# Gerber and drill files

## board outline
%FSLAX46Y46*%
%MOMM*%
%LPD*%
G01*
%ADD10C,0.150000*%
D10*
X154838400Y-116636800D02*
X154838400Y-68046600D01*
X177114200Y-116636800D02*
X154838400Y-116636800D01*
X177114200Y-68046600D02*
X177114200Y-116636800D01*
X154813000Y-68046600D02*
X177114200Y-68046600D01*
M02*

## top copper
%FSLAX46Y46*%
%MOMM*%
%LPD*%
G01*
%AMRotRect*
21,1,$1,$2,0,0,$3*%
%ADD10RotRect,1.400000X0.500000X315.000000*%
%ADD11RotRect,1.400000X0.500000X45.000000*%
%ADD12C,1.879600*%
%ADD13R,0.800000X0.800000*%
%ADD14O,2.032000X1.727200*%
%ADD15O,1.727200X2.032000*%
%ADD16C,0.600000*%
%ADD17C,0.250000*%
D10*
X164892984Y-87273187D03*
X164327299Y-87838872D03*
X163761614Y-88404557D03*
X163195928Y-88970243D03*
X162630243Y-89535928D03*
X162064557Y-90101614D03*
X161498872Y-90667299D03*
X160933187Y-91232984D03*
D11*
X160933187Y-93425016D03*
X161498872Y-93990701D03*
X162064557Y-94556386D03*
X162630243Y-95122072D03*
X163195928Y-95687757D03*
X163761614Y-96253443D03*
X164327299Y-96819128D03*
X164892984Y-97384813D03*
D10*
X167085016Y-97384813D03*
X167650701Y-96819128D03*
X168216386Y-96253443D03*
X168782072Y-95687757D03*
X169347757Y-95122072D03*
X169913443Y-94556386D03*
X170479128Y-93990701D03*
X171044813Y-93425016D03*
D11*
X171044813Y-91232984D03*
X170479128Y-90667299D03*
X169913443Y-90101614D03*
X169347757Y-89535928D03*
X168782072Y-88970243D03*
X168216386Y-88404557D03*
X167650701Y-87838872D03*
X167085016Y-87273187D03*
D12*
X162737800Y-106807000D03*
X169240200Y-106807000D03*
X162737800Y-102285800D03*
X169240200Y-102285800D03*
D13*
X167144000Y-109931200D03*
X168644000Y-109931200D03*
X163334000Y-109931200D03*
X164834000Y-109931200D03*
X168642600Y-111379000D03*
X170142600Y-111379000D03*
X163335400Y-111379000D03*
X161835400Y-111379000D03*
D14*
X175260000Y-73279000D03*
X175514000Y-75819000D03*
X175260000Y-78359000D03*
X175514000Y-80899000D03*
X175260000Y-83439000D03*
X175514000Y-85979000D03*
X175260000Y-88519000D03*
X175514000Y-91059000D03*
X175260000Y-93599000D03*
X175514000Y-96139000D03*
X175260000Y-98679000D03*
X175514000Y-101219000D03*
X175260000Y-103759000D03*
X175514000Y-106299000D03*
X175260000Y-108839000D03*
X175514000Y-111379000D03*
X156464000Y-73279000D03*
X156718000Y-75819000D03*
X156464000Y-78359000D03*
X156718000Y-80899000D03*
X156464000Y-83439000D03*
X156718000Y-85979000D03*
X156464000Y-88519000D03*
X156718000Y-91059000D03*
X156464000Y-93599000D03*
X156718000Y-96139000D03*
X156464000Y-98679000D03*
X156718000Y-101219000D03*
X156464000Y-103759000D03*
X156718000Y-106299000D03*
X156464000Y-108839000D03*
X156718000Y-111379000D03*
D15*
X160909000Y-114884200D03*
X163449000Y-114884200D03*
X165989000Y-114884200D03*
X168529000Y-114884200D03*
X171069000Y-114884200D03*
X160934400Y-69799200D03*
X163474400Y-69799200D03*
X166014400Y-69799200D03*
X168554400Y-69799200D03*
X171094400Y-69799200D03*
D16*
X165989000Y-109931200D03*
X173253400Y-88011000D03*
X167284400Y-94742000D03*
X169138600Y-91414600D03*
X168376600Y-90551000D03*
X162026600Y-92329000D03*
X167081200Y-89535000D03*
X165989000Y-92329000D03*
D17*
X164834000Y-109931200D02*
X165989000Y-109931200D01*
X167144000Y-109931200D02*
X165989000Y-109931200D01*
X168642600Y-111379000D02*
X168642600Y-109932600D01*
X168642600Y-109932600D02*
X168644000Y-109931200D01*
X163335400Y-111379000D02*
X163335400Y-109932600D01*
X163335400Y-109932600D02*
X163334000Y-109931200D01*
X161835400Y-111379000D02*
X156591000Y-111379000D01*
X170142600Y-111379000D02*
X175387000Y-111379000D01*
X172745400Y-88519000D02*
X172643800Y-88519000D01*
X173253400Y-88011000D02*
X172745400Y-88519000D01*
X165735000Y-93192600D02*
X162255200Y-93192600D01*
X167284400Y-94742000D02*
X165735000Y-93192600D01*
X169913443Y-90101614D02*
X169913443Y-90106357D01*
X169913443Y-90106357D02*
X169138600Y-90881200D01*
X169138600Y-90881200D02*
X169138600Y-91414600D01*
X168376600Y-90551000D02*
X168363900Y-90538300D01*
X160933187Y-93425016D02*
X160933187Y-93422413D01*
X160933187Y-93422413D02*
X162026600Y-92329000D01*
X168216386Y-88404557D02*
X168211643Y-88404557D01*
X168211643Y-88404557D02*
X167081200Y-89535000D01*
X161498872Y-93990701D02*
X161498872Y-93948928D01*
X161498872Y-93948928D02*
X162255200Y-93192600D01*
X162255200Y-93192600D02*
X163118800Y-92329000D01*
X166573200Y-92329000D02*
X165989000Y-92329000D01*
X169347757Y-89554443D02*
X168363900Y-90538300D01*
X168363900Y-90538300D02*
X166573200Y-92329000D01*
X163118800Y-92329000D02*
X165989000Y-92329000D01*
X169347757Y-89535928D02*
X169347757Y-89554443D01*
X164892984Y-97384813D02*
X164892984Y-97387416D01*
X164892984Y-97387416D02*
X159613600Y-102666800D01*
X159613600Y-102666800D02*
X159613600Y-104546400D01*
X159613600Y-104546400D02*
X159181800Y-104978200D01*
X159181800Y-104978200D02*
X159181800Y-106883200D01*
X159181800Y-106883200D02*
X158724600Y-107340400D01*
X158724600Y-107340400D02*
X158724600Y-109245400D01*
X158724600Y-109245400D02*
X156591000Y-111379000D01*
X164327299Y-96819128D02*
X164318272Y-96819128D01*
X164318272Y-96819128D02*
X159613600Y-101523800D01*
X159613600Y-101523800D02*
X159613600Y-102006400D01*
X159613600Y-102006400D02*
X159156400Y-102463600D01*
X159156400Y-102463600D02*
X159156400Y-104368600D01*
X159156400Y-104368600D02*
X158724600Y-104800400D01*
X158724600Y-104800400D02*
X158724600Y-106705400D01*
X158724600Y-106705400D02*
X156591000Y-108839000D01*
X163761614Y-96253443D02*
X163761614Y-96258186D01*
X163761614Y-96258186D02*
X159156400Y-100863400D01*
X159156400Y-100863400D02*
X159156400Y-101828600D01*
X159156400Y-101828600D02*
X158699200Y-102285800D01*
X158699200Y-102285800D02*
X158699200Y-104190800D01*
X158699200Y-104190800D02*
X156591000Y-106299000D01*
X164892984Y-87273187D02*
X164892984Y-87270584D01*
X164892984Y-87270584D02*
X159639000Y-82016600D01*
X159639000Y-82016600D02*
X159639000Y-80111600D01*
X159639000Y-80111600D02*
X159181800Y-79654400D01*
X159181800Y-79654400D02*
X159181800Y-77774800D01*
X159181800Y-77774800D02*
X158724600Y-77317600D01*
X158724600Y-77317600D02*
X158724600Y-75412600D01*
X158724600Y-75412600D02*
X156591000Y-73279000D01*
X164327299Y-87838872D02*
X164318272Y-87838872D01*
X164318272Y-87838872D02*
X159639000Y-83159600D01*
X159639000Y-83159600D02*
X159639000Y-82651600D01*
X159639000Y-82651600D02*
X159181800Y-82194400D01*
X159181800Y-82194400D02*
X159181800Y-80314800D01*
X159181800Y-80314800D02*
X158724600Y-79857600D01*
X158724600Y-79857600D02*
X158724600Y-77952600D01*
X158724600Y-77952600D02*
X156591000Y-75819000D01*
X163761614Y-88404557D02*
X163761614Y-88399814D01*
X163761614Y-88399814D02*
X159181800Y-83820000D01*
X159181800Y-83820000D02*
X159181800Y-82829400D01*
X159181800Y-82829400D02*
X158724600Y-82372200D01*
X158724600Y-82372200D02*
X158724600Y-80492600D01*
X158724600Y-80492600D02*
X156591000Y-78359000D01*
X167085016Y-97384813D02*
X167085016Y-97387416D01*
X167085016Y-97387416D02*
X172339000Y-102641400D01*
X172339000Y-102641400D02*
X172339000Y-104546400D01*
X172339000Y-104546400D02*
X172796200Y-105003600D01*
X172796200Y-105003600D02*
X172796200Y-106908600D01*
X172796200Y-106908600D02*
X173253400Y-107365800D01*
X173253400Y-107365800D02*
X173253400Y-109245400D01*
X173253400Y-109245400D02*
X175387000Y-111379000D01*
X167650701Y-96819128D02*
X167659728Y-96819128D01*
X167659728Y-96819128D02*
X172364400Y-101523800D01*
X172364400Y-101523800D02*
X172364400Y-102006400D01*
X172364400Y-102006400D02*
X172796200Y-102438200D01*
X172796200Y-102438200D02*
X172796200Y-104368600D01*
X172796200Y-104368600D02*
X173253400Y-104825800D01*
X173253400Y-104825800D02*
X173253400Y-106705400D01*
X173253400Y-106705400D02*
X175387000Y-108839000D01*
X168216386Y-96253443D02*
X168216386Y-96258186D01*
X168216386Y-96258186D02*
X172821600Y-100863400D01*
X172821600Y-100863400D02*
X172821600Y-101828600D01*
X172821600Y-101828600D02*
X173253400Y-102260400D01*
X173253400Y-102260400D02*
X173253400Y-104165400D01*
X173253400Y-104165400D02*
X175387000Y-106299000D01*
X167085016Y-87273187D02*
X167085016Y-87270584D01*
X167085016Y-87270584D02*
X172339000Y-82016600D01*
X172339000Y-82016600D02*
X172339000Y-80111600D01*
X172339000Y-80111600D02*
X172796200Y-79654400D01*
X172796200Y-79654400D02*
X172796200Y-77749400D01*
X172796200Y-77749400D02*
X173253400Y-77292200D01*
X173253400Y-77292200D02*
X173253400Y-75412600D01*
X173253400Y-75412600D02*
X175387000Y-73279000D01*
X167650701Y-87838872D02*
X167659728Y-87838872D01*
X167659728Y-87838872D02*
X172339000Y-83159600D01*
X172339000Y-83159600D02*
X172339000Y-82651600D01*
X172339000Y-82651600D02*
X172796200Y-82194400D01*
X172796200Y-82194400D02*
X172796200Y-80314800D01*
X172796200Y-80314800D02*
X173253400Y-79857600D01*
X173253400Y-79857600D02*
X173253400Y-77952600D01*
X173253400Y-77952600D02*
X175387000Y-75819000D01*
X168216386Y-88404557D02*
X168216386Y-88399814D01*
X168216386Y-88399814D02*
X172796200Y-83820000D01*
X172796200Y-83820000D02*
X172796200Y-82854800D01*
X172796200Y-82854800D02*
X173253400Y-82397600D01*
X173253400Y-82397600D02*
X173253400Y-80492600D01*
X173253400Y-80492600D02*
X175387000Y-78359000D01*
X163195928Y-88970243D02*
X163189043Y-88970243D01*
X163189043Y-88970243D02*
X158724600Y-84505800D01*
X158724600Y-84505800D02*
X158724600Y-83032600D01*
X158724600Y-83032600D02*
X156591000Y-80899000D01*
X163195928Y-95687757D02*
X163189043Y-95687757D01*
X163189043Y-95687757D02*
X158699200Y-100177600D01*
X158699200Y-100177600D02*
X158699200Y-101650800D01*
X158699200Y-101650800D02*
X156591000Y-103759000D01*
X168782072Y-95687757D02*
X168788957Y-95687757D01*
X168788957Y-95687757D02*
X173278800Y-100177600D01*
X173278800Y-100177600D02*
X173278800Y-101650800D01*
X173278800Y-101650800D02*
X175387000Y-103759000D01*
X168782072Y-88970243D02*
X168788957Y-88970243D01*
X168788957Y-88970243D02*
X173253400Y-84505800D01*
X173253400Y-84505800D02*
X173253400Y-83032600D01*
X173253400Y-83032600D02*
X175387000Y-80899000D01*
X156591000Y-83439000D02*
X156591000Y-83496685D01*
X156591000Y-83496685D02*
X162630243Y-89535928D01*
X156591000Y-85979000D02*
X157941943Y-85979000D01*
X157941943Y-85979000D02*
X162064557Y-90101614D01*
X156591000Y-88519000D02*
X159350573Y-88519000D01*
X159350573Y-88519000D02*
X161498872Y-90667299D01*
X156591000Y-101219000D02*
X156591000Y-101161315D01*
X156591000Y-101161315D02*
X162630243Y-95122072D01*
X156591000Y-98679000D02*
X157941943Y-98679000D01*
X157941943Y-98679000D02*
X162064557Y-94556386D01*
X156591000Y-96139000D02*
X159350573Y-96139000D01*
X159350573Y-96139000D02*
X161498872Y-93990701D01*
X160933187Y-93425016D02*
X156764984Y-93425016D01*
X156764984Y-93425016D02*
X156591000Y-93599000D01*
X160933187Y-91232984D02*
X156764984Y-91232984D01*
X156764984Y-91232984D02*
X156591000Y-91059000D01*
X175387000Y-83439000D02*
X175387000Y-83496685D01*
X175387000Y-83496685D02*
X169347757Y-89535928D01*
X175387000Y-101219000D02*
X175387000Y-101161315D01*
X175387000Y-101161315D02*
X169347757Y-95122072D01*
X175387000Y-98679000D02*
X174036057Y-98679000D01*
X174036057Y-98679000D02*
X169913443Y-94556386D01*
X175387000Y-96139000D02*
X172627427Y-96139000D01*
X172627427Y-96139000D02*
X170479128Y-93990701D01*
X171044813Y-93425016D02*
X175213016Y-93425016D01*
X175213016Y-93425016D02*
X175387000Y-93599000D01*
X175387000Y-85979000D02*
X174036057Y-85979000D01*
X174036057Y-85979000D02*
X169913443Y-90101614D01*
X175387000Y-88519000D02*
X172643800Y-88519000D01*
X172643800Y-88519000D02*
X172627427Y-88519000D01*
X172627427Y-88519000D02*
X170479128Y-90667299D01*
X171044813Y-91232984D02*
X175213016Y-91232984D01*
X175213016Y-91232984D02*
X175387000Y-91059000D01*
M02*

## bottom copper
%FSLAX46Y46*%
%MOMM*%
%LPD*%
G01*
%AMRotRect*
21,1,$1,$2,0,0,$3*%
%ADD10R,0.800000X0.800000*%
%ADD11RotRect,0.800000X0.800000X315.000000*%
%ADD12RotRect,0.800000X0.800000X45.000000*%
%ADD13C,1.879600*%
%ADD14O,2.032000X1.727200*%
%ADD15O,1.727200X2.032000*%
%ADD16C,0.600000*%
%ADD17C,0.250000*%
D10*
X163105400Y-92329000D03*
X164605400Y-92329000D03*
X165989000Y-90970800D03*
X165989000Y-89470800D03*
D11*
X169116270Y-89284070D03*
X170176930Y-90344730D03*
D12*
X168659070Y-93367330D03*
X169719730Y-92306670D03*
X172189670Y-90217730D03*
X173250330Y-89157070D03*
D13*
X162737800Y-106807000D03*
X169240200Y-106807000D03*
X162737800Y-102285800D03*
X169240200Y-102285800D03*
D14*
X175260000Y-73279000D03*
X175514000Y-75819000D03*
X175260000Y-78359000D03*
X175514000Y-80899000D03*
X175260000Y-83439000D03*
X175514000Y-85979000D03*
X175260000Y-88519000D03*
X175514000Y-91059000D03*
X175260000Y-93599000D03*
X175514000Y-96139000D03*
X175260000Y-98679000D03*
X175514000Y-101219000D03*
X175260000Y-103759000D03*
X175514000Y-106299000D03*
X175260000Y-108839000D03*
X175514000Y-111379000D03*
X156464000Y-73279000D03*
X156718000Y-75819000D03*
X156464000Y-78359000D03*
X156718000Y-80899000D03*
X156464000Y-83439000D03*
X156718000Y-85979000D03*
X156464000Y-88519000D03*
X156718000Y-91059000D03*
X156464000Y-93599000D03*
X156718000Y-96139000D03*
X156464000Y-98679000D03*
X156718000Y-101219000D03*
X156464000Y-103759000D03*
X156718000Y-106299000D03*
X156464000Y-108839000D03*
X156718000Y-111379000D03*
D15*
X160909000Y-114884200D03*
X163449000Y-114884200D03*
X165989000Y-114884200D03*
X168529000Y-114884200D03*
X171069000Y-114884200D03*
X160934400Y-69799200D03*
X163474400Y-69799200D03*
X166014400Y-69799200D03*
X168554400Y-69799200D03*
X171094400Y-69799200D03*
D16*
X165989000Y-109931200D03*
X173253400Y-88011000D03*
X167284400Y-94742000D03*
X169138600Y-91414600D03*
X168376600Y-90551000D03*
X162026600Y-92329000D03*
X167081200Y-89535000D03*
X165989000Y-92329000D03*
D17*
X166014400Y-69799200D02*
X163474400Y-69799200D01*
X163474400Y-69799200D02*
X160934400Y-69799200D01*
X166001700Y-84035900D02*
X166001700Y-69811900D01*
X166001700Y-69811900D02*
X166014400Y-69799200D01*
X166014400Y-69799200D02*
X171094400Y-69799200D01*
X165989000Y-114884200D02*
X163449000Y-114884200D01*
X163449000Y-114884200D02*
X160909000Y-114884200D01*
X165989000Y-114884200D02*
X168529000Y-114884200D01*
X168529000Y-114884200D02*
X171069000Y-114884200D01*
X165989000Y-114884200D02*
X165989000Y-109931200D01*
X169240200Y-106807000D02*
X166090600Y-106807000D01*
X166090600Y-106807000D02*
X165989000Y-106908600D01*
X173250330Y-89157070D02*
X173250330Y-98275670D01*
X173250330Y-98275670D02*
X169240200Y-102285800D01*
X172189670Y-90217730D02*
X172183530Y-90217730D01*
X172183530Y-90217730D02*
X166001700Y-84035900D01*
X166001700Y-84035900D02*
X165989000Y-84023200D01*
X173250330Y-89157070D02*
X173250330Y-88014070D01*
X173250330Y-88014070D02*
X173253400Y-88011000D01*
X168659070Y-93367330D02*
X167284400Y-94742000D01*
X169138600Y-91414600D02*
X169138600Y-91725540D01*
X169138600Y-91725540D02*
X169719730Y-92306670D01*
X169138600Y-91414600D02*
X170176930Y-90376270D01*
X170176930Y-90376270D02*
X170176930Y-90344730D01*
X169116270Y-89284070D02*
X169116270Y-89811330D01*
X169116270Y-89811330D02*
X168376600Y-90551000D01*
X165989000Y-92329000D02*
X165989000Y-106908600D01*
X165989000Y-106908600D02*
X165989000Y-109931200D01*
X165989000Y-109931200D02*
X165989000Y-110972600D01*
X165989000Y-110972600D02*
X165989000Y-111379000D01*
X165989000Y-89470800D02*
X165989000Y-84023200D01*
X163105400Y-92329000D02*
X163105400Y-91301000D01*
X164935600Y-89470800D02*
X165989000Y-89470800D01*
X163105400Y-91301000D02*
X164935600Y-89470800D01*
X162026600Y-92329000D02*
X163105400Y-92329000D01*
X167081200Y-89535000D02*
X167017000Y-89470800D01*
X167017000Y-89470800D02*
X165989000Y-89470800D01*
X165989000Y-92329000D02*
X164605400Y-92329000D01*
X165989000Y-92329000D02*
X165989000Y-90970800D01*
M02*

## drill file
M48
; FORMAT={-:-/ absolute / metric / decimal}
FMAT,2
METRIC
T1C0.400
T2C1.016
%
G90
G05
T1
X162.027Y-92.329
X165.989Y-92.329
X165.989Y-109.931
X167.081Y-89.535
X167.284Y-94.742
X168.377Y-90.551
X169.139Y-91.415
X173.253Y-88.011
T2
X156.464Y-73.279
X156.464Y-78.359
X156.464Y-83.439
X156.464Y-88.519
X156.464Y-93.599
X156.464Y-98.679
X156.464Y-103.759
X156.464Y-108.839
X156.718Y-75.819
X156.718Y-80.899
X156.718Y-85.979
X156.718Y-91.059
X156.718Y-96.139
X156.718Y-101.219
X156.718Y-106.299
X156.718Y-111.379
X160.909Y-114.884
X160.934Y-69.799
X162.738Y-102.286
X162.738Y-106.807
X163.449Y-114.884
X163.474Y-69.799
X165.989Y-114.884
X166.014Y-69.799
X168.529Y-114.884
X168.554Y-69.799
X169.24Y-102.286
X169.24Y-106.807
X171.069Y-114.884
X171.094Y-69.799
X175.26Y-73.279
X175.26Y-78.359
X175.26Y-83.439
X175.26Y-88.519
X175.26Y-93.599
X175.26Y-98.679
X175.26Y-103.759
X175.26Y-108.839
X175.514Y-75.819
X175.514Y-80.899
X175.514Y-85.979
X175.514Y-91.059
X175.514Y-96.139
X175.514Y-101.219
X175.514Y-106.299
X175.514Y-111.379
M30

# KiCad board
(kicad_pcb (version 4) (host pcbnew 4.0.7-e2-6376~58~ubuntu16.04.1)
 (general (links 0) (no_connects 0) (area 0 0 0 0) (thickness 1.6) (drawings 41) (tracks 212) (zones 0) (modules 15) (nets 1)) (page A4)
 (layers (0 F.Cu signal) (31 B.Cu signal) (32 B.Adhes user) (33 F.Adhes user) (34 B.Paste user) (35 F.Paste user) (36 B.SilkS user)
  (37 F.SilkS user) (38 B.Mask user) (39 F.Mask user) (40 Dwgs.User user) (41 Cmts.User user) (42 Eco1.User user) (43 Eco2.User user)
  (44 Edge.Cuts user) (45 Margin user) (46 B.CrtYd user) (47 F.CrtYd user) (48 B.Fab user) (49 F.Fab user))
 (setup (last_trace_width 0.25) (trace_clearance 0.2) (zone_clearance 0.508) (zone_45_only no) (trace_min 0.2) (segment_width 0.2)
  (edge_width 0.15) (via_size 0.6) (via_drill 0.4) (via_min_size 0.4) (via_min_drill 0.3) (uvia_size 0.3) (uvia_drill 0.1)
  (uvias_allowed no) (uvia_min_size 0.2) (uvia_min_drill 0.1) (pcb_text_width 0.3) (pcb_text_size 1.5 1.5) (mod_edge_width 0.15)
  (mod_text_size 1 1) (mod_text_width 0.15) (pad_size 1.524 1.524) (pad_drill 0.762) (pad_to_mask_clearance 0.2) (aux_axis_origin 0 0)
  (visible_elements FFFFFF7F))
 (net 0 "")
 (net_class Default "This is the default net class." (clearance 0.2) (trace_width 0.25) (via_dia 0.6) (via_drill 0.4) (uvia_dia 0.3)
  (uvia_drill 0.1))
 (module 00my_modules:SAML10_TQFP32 (layer F.Cu) (at 165.989 92.329 315)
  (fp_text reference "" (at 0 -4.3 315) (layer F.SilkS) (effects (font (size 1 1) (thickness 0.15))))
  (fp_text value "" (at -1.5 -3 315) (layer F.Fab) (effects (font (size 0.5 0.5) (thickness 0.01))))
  (pad PA00 smd rect (at -4.35 -2.8 315) (size 1.4 0.5) (layers F.Cu F.Paste F.Mask))
  (pad PA01 smd rect (at -4.35 -2 315) (size 1.4 0.5) (layers F.Cu F.Paste F.Mask))
  (pad PA02 smd rect (at -4.35 -1.2 315) (size 1.4 0.5) (layers F.Cu F.Paste F.Mask))
  (pad PA03 smd rect (at -4.35 -0.4 315) (size 1.4 0.5) (layers F.Cu F.Paste F.Mask))
  (pad PA04 smd rect (at -4.35 0.4 315) (size 1.4 0.5) (layers F.Cu F.Paste F.Mask))
  (pad PA05 smd rect (at -4.35 1.2 315) (size 1.4 0.5) (layers F.Cu F.Paste F.Mask))
  (pad PA06 smd rect (at -4.35 2 315) (size 1.4 0.5) (layers F.Cu F.Paste F.Mask))
  (pad PA07 smd rect (at -4.35 2.8 315) (size 1.4 0.5) (layers F.Cu F.Paste F.Mask))
  (pad VDDA smd rect (at -2.8 4.35 45) (size 1.4 0.5) (layers F.Cu F.Paste F.Mask))
  (pad GNDA smd rect (at -2 4.35 45) (size 1.4 0.5) (layers F.Cu F.Paste F.Mask))
  (pad PA08 smd rect (at -1.2 4.35 45) (size 1.4 0.5) (layers F.Cu F.Paste F.Mask))
  (pad PA09 smd rect (at -0.4 4.35 45) (size 1.4 0.5) (layers F.Cu F.Paste F.Mask))
  (pad PA10 smd rect (at 0.4 4.35 45) (size 1.4 0.5) (layers F.Cu F.Paste F.Mask))
  (pad PA11 smd rect (at 1.2 4.35 45) (size 1.4 0.5) (layers F.Cu F.Paste F.Mask))
  (pad PA14 smd rect (at 2 4.35 45) (size 1.4 0.5) (layers F.Cu F.Paste F.Mask))
  (pad PA15 smd rect (at 2.8 4.35 45) (size 1.4 0.5) (layers F.Cu F.Paste F.Mask))
  (pad PA16 smd rect (at 4.35 2.8 315) (size 1.4 0.5) (layers F.Cu F.Paste F.Mask))
  (pad PA17 smd rect (at 4.35 2 315) (size 1.4 0.5) (layers F.Cu F.Paste F.Mask))
  (pad PA18 smd rect (at 4.35 1.2 315) (size 1.4 0.5) (layers F.Cu F.Paste F.Mask))
  (pad PA19 smd rect (at 4.35 0.4 315) (size 1.4 0.5) (layers F.Cu F.Paste F.Mask))
  (pad PA22 smd rect (at 4.35 -0.4 315) (size 1.4 0.5) (layers F.Cu F.Paste F.Mask))
  (pad PA23 smd rect (at 4.35 -1.2 315) (size 1.4 0.5) (layers F.Cu F.Paste F.Mask))
  (pad PA24 smd rect (at 4.35 -2 315) (size 1.4 0.5) (layers F.Cu F.Paste F.Mask))
  (pad PA25 smd rect (at 4.35 -2.8 315) (size 1.4 0.5) (layers F.Cu F.Paste F.Mask))
  (pad PA27 smd rect (at 2.8 -4.35 45) (size 1.4 0.5) (layers F.Cu F.Paste F.Mask))
  (pad RSTN smd rect (at 2 -4.35 45) (size 1.4 0.5) (layers F.Cu F.Paste F.Mask))
  (pad VCOR smd rect (at 1.2 -4.35 45) (size 1.4 0.5) (layers F.Cu F.Paste F.Mask))
  (pad GND smd rect (at 0.4 -4.35 45) (size 1.4 0.5) (layers F.Cu F.Paste F.Mask))
  (pad VOUT smd rect (at -0.4 -4.35 45) (size 1.4 0.5) (layers F.Cu F.Paste F.Mask))
  (pad VIO smd rect (at -1.2 -4.35 45) (size 1.4 0.5) (layers F.Cu F.Paste F.Mask))
  (pad CLK smd rect (at -2 -4.35 45) (size 1.4 0.5) (layers F.Cu F.Paste F.Mask))
  (pad DIO smd rect (at -2.8 -4.35 45) (size 1.4 0.5) (layers F.Cu F.Paste F.Mask)))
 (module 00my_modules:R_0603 (layer B.Cu) (at 163.8554 92.329)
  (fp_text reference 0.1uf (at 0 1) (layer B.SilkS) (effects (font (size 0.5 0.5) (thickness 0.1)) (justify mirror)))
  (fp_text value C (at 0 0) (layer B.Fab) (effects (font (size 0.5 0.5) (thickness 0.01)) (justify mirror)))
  (pad 1 smd rect (at -0.75 0) (size 0.8 0.8) (layers B.Cu B.Paste B.Mask))
  (pad 2 smd rect (at 0.75 0) (size 0.8 0.8) (layers B.Cu B.Paste B.Mask)))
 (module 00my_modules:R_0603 (layer B.Cu) (at 165.989 90.2208 90)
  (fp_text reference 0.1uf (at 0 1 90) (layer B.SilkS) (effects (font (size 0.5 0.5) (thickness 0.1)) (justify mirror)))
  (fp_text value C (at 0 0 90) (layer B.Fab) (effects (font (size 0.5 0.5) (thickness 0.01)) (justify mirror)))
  (pad 1 smd rect (at -0.75 0 90) (size 0.8 0.8) (layers B.Cu B.Paste B.Mask))
  (pad 2 smd rect (at 0.75 0 90) (size 0.8 0.8) (layers B.Cu B.Paste B.Mask)))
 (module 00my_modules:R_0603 (layer B.Cu) (at 169.6466 89.8144 315)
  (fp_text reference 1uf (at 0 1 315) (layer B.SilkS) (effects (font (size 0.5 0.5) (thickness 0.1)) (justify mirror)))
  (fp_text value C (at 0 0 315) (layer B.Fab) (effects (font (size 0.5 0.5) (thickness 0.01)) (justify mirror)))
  (pad 1 smd rect (at -0.75 0 315) (size 0.8 0.8) (layers B.Cu B.Paste B.Mask))
  (pad 2 smd rect (at 0.75 0 315) (size 0.8 0.8) (layers B.Cu B.Paste B.Mask)))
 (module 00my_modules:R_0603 (layer B.Cu) (at 169.1894 92.837 45)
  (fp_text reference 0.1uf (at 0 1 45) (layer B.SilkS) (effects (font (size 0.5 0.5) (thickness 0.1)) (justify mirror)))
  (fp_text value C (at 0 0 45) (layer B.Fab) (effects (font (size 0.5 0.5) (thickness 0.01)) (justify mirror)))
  (pad 1 smd rect (at -0.75 0 45) (size 0.8 0.8) (layers B.Cu B.Paste B.Mask))
  (pad 2 smd rect (at 0.75 0 45) (size 0.8 0.8) (layers B.Cu B.Paste B.Mask)))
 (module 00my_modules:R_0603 (layer B.Cu) (at 172.72 89.6874 45)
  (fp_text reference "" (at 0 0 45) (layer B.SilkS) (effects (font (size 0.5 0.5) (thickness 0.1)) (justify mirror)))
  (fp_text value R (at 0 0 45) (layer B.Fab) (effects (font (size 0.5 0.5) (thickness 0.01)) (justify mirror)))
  (pad 1 smd rect (at -0.75 0 45) (size 0.8 0.8) (layers B.Cu B.Paste B.Mask))
  (pad 2 smd rect (at 0.75 0 45) (size 0.8 0.8) (layers B.Cu B.Paste B.Mask)))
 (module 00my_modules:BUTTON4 (layer F.Cu) (at 165.989 104.5464)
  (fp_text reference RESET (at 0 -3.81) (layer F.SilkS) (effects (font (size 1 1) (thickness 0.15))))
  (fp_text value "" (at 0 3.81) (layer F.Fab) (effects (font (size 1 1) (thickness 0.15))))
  (pad 1 thru_hole circle (at -3.2512 2.2606) (size 1.8796 1.8796) (drill 1.016) (layers *.Cu *.Mask F.SilkS))
  (pad 2 thru_hole circle (at 3.2512 2.2606) (size 1.8796 1.8796) (drill 1.016) (layers *.Cu *.Mask F.SilkS))
  (pad 3 thru_hole circle (at -3.2512 -2.2606) (size 1.8796 1.8796) (drill 1.016) (layers *.Cu *.Mask F.SilkS))
  (pad 4 thru_hole circle (at 3.2512 -2.2606) (size 1.8796 1.8796) (drill 1.016) (layers *.Cu *.Mask F.SilkS)))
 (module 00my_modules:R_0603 (layer F.Cu) (at 167.894 109.9312)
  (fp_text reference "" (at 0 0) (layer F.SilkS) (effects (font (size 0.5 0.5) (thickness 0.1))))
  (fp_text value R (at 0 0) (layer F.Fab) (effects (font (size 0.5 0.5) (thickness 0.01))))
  (pad 1 smd rect (at -0.75 0) (size 0.8 0.8) (layers F.Cu F.Paste F.Mask))
  (pad 2 smd rect (at 0.75 0) (size 0.8 0.8) (layers F.Cu F.Paste F.Mask)))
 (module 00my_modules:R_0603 (layer F.Cu) (at 164.084 109.9312)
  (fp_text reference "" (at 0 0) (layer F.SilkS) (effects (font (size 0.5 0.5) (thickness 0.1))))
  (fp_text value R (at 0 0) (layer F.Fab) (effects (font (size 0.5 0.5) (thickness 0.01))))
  (pad 1 smd rect (at -0.75 0) (size 0.8 0.8) (layers F.Cu F.Paste F.Mask))
  (pad 2 smd rect (at 0.75 0) (size 0.8 0.8) (layers F.Cu F.Paste F.Mask)))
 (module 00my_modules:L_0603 (layer F.Cu) (at 169.3926 111.379)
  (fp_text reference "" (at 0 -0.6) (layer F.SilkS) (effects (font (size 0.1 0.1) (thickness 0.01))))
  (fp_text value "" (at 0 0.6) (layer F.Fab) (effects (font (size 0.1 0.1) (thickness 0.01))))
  (pad 1 smd rect (at -0.75 0) (size 0.8 0.8) (layers F.Cu F.Paste F.Mask))
  (pad 2 smd rect (at 0.75 0) (size 0.8 0.8) (layers F.Cu F.Paste F.Mask)))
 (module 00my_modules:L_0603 (layer F.Cu) (at 162.5854 111.379 180)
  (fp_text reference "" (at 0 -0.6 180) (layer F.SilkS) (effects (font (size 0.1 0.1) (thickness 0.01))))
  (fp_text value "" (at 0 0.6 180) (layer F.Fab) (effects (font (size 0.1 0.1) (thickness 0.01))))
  (pad 1 smd rect (at -0.75 0 180) (size 0.8 0.8) (layers F.Cu F.Paste F.Mask))
  (pad 2 smd rect (at 0.75 0 180) (size 0.8 0.8) (layers F.Cu F.Paste F.Mask)))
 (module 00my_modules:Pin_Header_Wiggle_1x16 (layer F.Cu) (at 175.387 73.279)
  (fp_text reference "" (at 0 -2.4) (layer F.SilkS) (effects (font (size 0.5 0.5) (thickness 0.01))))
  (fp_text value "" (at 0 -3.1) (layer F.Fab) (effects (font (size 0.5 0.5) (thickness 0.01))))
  (pad 1 thru_hole oval (at -0.127 0) (size 2.032 1.7272) (drill 1.016) (layers *.Cu *.Mask F.SilkS))
  (pad 2 thru_hole oval (at 0.127 2.54) (size 2.032 1.7272) (drill 1.016) (layers *.Cu *.Mask F.SilkS))
  (pad 3 thru_hole oval (at -0.127 5.08) (size 2.032 1.7272) (drill 1.016) (layers *.Cu *.Mask F.SilkS))
  (pad 4 thru_hole oval (at 0.127 7.62) (size 2.032 1.7272) (drill 1.016) (layers *.Cu *.Mask F.SilkS))
  (pad 5 thru_hole oval (at -0.127 10.16) (size 2.032 1.7272) (drill 1.016) (layers *.Cu *.Mask F.SilkS))
  (pad 6 thru_hole oval (at 0.127 12.7) (size 2.032 1.7272) (drill 1.016) (layers *.Cu *.Mask F.SilkS))
  (pad 7 thru_hole oval (at -0.127 15.24) (size 2.032 1.7272) (drill 1.016) (layers *.Cu *.Mask F.SilkS))
  (pad 8 thru_hole oval (at 0.127 17.78) (size 2.032 1.7272) (drill 1.016) (layers *.Cu *.Mask F.SilkS))
  (pad 9 thru_hole oval (at -0.127 20.32) (size 2.032 1.7272) (drill 1.016) (layers *.Cu *.Mask F.SilkS))
  (pad 10 thru_hole oval (at 0.127 22.86) (size 2.032 1.7272) (drill 1.016) (layers *.Cu *.Mask F.SilkS))
  (pad 11 thru_hole oval (at -0.127 25.4) (size 2.032 1.7272) (drill 1.016) (layers *.Cu *.Mask F.SilkS))
  (pad 12 thru_hole oval (at 0.127 27.94) (size 2.032 1.7272) (drill 1.016) (layers *.Cu *.Mask F.SilkS))
  (pad 13 thru_hole oval (at -0.127 30.48) (size 2.032 1.7272) (drill 1.016) (layers *.Cu *.Mask F.SilkS))
  (pad 14 thru_hole oval (at 0.127 33.02) (size 2.032 1.7272) (drill 1.016) (layers *.Cu *.Mask F.SilkS))
  (pad 15 thru_hole oval (at -0.127 35.56) (size 2.032 1.7272) (drill 1.016) (layers *.Cu *.Mask F.SilkS))
  (pad 16 thru_hole oval (at 0.127 38.1) (size 2.032 1.7272) (drill 1.016) (layers *.Cu *.Mask F.SilkS)))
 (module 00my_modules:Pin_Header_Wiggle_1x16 (layer F.Cu) (at 156.591 73.279)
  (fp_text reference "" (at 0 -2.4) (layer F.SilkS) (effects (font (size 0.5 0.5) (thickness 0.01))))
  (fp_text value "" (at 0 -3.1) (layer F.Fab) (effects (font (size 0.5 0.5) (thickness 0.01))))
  (pad 1 thru_hole oval (at -0.127 0) (size 2.032 1.7272) (drill 1.016) (layers *.Cu *.Mask F.SilkS))
  (pad 2 thru_hole oval (at 0.127 2.54) (size 2.032 1.7272) (drill 1.016) (layers *.Cu *.Mask F.SilkS))
  (pad 3 thru_hole oval (at -0.127 5.08) (size 2.032 1.7272) (drill 1.016) (layers *.Cu *.Mask F.SilkS))
  (pad 4 thru_hole oval (at 0.127 7.62) (size 2.032 1.7272) (drill 1.016) (layers *.Cu *.Mask F.SilkS))
  (pad 5 thru_hole oval (at -0.127 10.16) (size 2.032 1.7272) (drill 1.016) (layers *.Cu *.Mask F.SilkS))
  (pad 6 thru_hole oval (at 0.127 12.7) (size 2.032 1.7272) (drill 1.016) (layers *.Cu *.Mask F.SilkS))
  (pad 7 thru_hole oval (at -0.127 15.24) (size 2.032 1.7272) (drill 1.016) (layers *.Cu *.Mask F.SilkS))
  (pad 8 thru_hole oval (at 0.127 17.78) (size 2.032 1.7272) (drill 1.016) (layers *.Cu *.Mask F.SilkS))
  (pad 9 thru_hole oval (at -0.127 20.32) (size 2.032 1.7272) (drill 1.016) (layers *.Cu *.Mask F.SilkS))
  (pad 10 thru_hole oval (at 0.127 22.86) (size 2.032 1.7272) (drill 1.016) (layers *.Cu *.Mask F.SilkS))
  (pad 11 thru_hole oval (at -0.127 25.4) (size 2.032 1.7272) (drill 1.016) (layers *.Cu *.Mask F.SilkS))
  (pad 12 thru_hole oval (at 0.127 27.94) (size 2.032 1.7272) (drill 1.016) (layers *.Cu *.Mask F.SilkS))
  (pad 13 thru_hole oval (at -0.127 30.48) (size 2.032 1.7272) (drill 1.016) (layers *.Cu *.Mask F.SilkS))
  (pad 14 thru_hole oval (at 0.127 33.02) (size 2.032 1.7272) (drill 1.016) (layers *.Cu *.Mask F.SilkS))
  (pad 15 thru_hole oval (at -0.127 35.56) (size 2.032 1.7272) (drill 1.016) (layers *.Cu *.Mask F.SilkS))
  (pad 16 thru_hole oval (at 0.127 38.1) (size 2.032 1.7272) (drill 1.016) (layers *.Cu *.Mask F.SilkS)))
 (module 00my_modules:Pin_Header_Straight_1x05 (layer F.Cu) (at 160.909 114.8842 90)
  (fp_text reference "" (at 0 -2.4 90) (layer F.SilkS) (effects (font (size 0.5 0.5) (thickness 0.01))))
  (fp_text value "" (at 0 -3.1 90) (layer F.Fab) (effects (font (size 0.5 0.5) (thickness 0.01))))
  (pad 1 thru_hole oval (at 0 0 90) (size 2.032 1.7272) (drill 1.016) (layers *.Cu *.Mask F.SilkS))
  (pad 2 thru_hole oval (at 0 2.54 90) (size 2.032 1.7272) (drill 1.016) (layers *.Cu *.Mask F.SilkS))
  (pad 3 thru_hole oval (at 0 5.08 90) (size 2.032 1.7272) (drill 1.016) (layers *.Cu *.Mask F.SilkS))
  (pad 4 thru_hole oval (at 0 7.62 90) (size 2.032 1.7272) (drill 1.016) (layers *.Cu *.Mask F.SilkS))
  (pad 5 thru_hole oval (at 0 10.16 90) (size 2.032 1.7272) (drill 1.016) (layers *.Cu *.Mask F.SilkS)))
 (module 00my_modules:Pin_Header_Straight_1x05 (layer F.Cu) (at 160.9344 69.7992 90)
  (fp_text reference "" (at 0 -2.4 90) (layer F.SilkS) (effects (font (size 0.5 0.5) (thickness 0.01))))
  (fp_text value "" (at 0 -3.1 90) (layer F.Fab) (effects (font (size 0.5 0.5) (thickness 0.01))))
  (pad 1 thru_hole oval (at 0 0 90) (size 2.032 1.7272) (drill 1.016) (layers *.Cu *.Mask F.SilkS))
  (pad 2 thru_hole oval (at 0 2.54 90) (size 2.032 1.7272) (drill 1.016) (layers *.Cu *.Mask F.SilkS))
  (pad 3 thru_hole oval (at 0 5.08 90) (size 2.032 1.7272) (drill 1.016) (layers *.Cu *.Mask F.SilkS))
  (pad 4 thru_hole oval (at 0 7.62 90) (size 2.032 1.7272) (drill 1.016) (layers *.Cu *.Mask F.SilkS))
  (pad 5 thru_hole oval (at 0 10.16 90) (size 2.032 1.7272) (drill 1.016) (layers *.Cu *.Mask F.SilkS)))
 (gr_line (start 154.8384 116.6368) (end 154.8384 68.0466) (angle 90) (layer Edge.Cuts) (width 0.15))
 (gr_line (start 177.1142 116.6368) (end 154.8384 116.6368) (angle 90) (layer Edge.Cuts) (width 0.15))
 (gr_line (start 177.1142 68.0466) (end 177.1142 116.6368) (angle 90) (layer Edge.Cuts) (width 0.15))
 (gr_line (start 154.813 68.0466) (end 177.1142 68.0466) (angle 90) (layer Edge.Cuts) (width 0.15))
 (segment (start 166.0144 69.7992) (end 163.4744 69.7992) (width 0.25) (layer B.Cu) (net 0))
 (segment (start 163.4744 69.7992) (end 160.9344 69.7992) (width 0.25) (layer B.Cu) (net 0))
 (segment (start 166.0017 84.0359) (end 166.0017 69.8119) (width 0.25) (layer B.Cu) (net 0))
 (segment (start 166.0017 69.8119) (end 166.0144 69.7992) (width 0.25) (layer B.Cu) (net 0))
 (segment (start 166.0144 69.7992) (end 171.0944 69.7992) (width 0.25) (layer B.Cu) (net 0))
 (segment (start 165.989 114.8842) (end 163.449 114.8842) (width 0.25) (layer B.Cu) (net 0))
 (segment (start 163.449 114.8842) (end 160.909 114.8842) (width 0.25) (layer B.Cu) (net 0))
 (segment (start 165.989 114.8842) (end 168.529 114.8842) (width 0.25) (layer B.Cu) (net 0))
 (segment (start 168.529 114.8842) (end 171.069 114.8842) (width 0.25) (layer B.Cu) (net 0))
 (segment (start 165.989 114.8842) (end 165.989 109.9312) (width 0.25) (layer B.Cu) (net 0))
 (segment (start 164.834 109.9312) (end 165.989 109.9312) (width 0.25) (layer F.Cu) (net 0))
 (segment (start 167.144 109.9312) (end 165.989 109.9312) (width 0.25) (layer F.Cu) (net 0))
 (via (at 165.989 109.9312) (size 0.6) (drill 0.4) (layers F.Cu B.Cu) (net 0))
 (segment (start 168.6426 111.379) (end 168.6426 109.9326) (width 0.25) (layer F.Cu) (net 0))
 (segment (start 168.6426 109.9326) (end 168.644 109.9312) (width 0.25) (layer F.Cu) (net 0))
 (segment (start 163.3354 111.379) (end 163.3354 109.9326) (width 0.25) (layer F.Cu) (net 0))
 (segment (start 163.3354 109.9326) (end 163.334 109.9312) (width 0.25) (layer F.Cu) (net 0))
 (segment (start 161.8354 111.379) (end 156.591 111.379) (width 0.25) (layer F.Cu) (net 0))
 (segment (start 170.1426 111.379) (end 175.387 111.379) (width 0.25) (layer F.Cu) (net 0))
 (segment (start 169.2402 106.807) (end 166.0906 106.807) (width 0.25) (layer B.Cu) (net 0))
 (segment (start 166.0906 106.807) (end 165.989 106.9086) (width 0.25) (layer B.Cu) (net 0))
 (segment (start 173.25033 89.15707) (end 173.25033 98.27567) (width 0.25) (layer B.Cu) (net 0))
 (segment (start 173.25033 98.27567) (end 169.2402 102.2858) (width 0.25) (layer B.Cu) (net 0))
 (segment (start 172.18967 90.21773) (end 172.18353 90.21773) (width 0.25) (layer B.Cu) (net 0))
 (segment (start 172.18353 90.21773) (end 166.0017 84.0359) (width 0.25) (layer B.Cu) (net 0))
 (segment (start 166.0017 84.0359) (end 165.989 84.0232) (width 0.25) (layer B.Cu) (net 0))
 (segment (start 173.25033 89.15707) (end 173.25033 88.01407) (width 0.25) (layer B.Cu) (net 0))
 (segment (start 172.7454 88.519) (end 172.6438 88.519) (width 0.25) (layer F.Cu) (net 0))
 (segment (start 173.2534 88.011) (end 172.7454 88.519) (width 0.25) (layer F.Cu) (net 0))
 (via (at 173.2534 88.011) (size 0.6) (drill 0.4) (layers F.Cu B.Cu) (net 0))
 (segment (start 173.25033 88.01407) (end 173.2534 88.011) (width 0.25) (layer B.Cu) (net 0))
 (segment (start 168.65907 93.36733) (end 167.2844 94.742) (width 0.25) (layer B.Cu) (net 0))
 (segment (start 165.735 93.1926) (end 162.2552 93.1926) (width 0.25) (layer F.Cu) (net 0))
 (segment (start 167.2844 94.742) (end 165.735 93.1926) (width 0.25) (layer F.Cu) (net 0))
 (via (at 167.2844 94.742) (size 0.6) (drill 0.4) (layers F.Cu B.Cu) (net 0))
 (segment (start 169.1386 91.4146) (end 169.1386 91.72554) (width 0.25) (layer B.Cu) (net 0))
 (segment (start 169.1386 91.72554) (end 169.71973 92.30667) (width 0.25) (layer B.Cu) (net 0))
 (segment (start 169.913443 90.101614) (end 169.913443 90.106357) (width 0.25) (layer F.Cu) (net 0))
 (segment (start 169.913443 90.106357) (end 169.1386 90.8812) (width 0.25) (layer F.Cu) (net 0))
 (segment (start 169.1386 91.4146) (end 170.17693 90.37627) (width 0.25) (layer B.Cu) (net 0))
 (via (at 169.1386 91.4146) (size 0.6) (drill 0.4) (layers F.Cu B.Cu) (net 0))
 (segment (start 169.1386 90.8812) (end 169.1386 91.4146) (width 0.25) (layer F.Cu) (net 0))
 (segment (start 170.17693 90.37627) (end 170.17693 90.34473) (width 0.25) (layer B.Cu) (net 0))
 (segment (start 169.11627 89.28407) (end 169.11627 89.81133) (width 0.25) (layer B.Cu) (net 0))
 (segment (start 169.11627 89.81133) (end 168.3766 90.551) (width 0.25) (layer B.Cu) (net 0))
 (via (at 168.3766 90.551) (size 0.6) (drill 0.4) (layers F.Cu B.Cu) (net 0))
 (segment (start 168.3766 90.551) (end 168.3639 90.5383) (width 0.25) (layer F.Cu) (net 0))
 (segment (start 165.989 92.329) (end 165.989 106.9086) (width 0.25) (layer B.Cu) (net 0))
 (segment (start 165.989 106.9086) (end 165.989 109.9312) (width 0.25) (layer B.Cu) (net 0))
 (segment (start 165.989 109.9312) (end 165.989 110.9726) (width 0.25) (layer B.Cu) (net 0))
 (segment (start 165.989 110.9726) (end 165.989 111.379) (width 0.25) (layer B.Cu) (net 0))
 (segment (start 165.989 89.4708) (end 165.989 84.0232) (width 0.25) (layer B.Cu) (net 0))
 (segment (start 163.1054 92.329) (end 163.1054 91.301) (width 0.25) (layer B.Cu) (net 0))
 (segment (start 164.9356 89.4708) (end 165.989 89.4708) (width 0.25) (layer B.Cu) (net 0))
 (segment (start 163.1054 91.301) (end 164.9356 89.4708) (width 0.25) (layer B.Cu) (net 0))
 (segment (start 160.933187 93.425016) (end 160.933187 93.422413) (width 0.25) (layer F.Cu) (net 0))
 (segment (start 160.933187 93.422413) (end 162.0266 92.329) (width 0.25) (layer F.Cu) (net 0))
 (segment (start 162.0266 92.329) (end 163.1054 92.329) (width 0.25) (layer B.Cu) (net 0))
 (via (at 162.0266 92.329) (size 0.6) (drill 0.4) (layers F.Cu B.Cu) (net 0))
 (segment (start 168.216386 88.404557) (end 168.211643 88.404557) (width 0.25) (layer F.Cu) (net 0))
 (segment (start 168.211643 88.404557) (end 167.0812 89.535) (width 0.25) (layer F.Cu) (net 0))
 (via (at 167.0812 89.535) (size 0.6) (drill 0.4) (layers F.Cu B.Cu) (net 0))
 (segment (start 167.0812 89.535) (end 167.017 89.4708) (width 0.25) (layer B.Cu) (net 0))
 (segment (start 167.017 89.4708) (end 165.989 89.4708) (width 0.25) (layer B.Cu) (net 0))
 (segment (start 165.989 92.329) (end 164.6054 92.329) (width 0.25) (layer B.Cu) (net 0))
 (segment (start 165.989 92.329) (end 165.989 90.9708) (width 0.25) (layer B.Cu) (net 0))
 (via (at 165.989 92.329) (size 0.6) (drill 0.4) (layers F.Cu B.Cu) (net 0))
 (segment (start 161.498872 93.990701) (end 161.498872 93.948928) (width 0.25) (layer F.Cu) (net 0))
 (segment (start 161.498872 93.948928) (end 162.2552 93.1926) (width 0.25) (layer F.Cu) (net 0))
 (segment (start 162.2552 93.1926) (end 163.1188 92.329) (width 0.25) (layer F.Cu) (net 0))
 (segment (start 166.5732 92.329) (end 165.989 92.329) (width 0.25) (layer F.Cu) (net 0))
 (segment (start 169.347757 89.554443) (end 168.3639 90.5383) (width 0.25) (layer F.Cu) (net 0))
 (segment (start 168.3639 90.5383) (end 166.5732 92.329) (width 0.25) (layer F.Cu) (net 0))
 (segment (start 163.1188 92.329) (end 165.989 92.329) (width 0.25) (layer F.Cu) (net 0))
 (segment (start 169.347757 89.535928) (end 169.347757 89.554443) (width 0.25) (layer F.Cu) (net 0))
 (segment (start 164.892984 97.384813) (end 164.892984 97.387416) (width 0.25) (layer F.Cu) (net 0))
 (segment (start 164.892984 97.387416) (end 159.6136 102.6668) (width 0.25) (layer F.Cu) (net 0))
 (segment (start 159.6136 102.6668) (end 159.6136 104.5464) (width 0.25) (layer F.Cu) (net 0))
 (segment (start 159.6136 104.5464) (end 159.1818 104.9782) (width 0.25) (layer F.Cu) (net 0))
 (segment (start 159.1818 104.9782) (end 159.1818 106.8832) (width 0.25) (layer F.Cu) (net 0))
 (segment (start 159.1818 106.8832) (end 158.7246 107.3404) (width 0.25) (layer F.Cu) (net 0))
 (segment (start 158.7246 107.3404) (end 158.7246 109.2454) (width 0.25) (layer F.Cu) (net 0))
 (segment (start 158.7246 109.2454) (end 156.591 111.379) (width 0.25) (layer F.Cu) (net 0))
 (segment (start 164.327299 96.819128) (end 164.318272 96.819128) (width 0.25) (layer F.Cu) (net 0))
 (segment (start 164.318272 96.819128) (end 159.6136 101.5238) (width 0.25) (layer F.Cu) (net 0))
 (segment (start 159.6136 101.5238) (end 159.6136 102.0064) (width 0.25) (layer F.Cu) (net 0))
 (segment (start 159.6136 102.0064) (end 159.1564 102.4636) (width 0.25) (layer F.Cu) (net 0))
 (segment (start 159.1564 102.4636) (end 159.1564 104.3686) (width 0.25) (layer F.Cu) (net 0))
 (segment (start 159.1564 104.3686) (end 158.7246 104.8004) (width 0.25) (layer F.Cu) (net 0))
 (segment (start 158.7246 104.8004) (end 158.7246 106.7054) (width 0.25) (layer F.Cu) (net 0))
 (segment (start 158.7246 106.7054) (end 156.591 108.839) (width 0.25) (layer F.Cu) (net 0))
 (segment (start 163.761614 96.253443) (end 163.761614 96.258186) (width 0.25) (layer F.Cu) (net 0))
 (segment (start 163.761614 96.258186) (end 159.1564 100.8634) (width 0.25) (layer F.Cu) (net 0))
 (segment (start 159.1564 100.8634) (end 159.1564 101.8286) (width 0.25) (layer F.Cu) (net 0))
 (segment (start 159.1564 101.8286) (end 158.6992 102.2858) (width 0.25) (layer F.Cu) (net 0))
 (segment (start 158.6992 102.2858) (end 158.6992 104.1908) (width 0.25) (layer F.Cu) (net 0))
 (segment (start 158.6992 104.1908) (end 156.591 106.299) (width 0.25) (layer F.Cu) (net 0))
 (segment (start 164.892984 87.273187) (end 164.892984 87.270584) (width 0.25) (layer F.Cu) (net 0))
 (segment (start 164.892984 87.270584) (end 159.639 82.0166) (width 0.25) (layer F.Cu) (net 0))
 (segment (start 159.639 82.0166) (end 159.639 80.1116) (width 0.25) (layer F.Cu) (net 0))
 (segment (start 159.639 80.1116) (end 159.1818 79.6544) (width 0.25) (layer F.Cu) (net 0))
 (segment (start 159.1818 79.6544) (end 159.1818 77.7748) (width 0.25) (layer F.Cu) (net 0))
 (segment (start 159.1818 77.7748) (end 158.7246 77.3176) (width 0.25) (layer F.Cu) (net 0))
 (segment (start 158.7246 77.3176) (end 158.7246 75.4126) (width 0.25) (layer F.Cu) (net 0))
 (segment (start 158.7246 75.4126) (end 156.591 73.279) (width 0.25) (layer F.Cu) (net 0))
 (segment (start 164.327299 87.838872) (end 164.318272 87.838872) (width 0.25) (layer F.Cu) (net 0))
 (segment (start 164.318272 87.838872) (end 159.639 83.1596) (width 0.25) (layer F.Cu) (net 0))
 (segment (start 159.639 83.1596) (end 159.639 82.6516) (width 0.25) (layer F.Cu) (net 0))
 (segment (start 159.639 82.6516) (end 159.1818 82.1944) (width 0.25) (layer F.Cu) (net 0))
 (segment (start 159.1818 82.1944) (end 159.1818 80.3148) (width 0.25) (layer F.Cu) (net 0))
 (segment (start 159.1818 80.3148) (end 158.7246 79.8576) (width 0.25) (layer F.Cu) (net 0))
 (segment (start 158.7246 79.8576) (end 158.7246 77.9526) (width 0.25) (layer F.Cu) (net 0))
 (segment (start 158.7246 77.9526) (end 156.591 75.819) (width 0.25) (layer F.Cu) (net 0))
 (segment (start 163.761614 88.404557) (end 163.761614 88.399814) (width 0.25) (layer F.Cu) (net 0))
 (segment (start 163.761614 88.399814) (end 159.1818 83.82) (width 0.25) (layer F.Cu) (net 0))
 (segment (start 159.1818 83.82) (end 159.1818 82.8294) (width 0.25) (layer F.Cu) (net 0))
 (segment (start 159.1818 82.8294) (end 158.7246 82.3722) (width 0.25) (layer F.Cu) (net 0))
 (segment (start 158.7246 82.3722) (end 158.7246 80.4926) (width 0.25) (layer F.Cu) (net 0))
 (segment (start 158.7246 80.4926) (end 156.591 78.359) (width 0.25) (layer F.Cu) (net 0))
 (segment (start 167.085016 97.384813) (end 167.085016 97.387416) (width 0.25) (layer F.Cu) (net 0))
 (segment (start 167.085016 97.387416) (end 172.339 102.6414) (width 0.25) (layer F.Cu) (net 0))
 (segment (start 172.339 102.6414) (end 172.339 104.5464) (width 0.25) (layer F.Cu) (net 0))
 (segment (start 172.339 104.5464) (end 172.7962 105.0036) (width 0.25) (layer F.Cu) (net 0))
 (segment (start 172.7962 105.0036) (end 172.7962 106.9086) (width 0.25) (layer F.Cu) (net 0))
 (segment (start 172.7962 106.9086) (end 173.2534 107.3658) (width 0.25) (layer F.Cu) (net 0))
 (segment (start 173.2534 107.3658) (end 173.2534 109.2454) (width 0.25) (layer F.Cu) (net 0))
 (segment (start 173.2534 109.2454) (end 175.387 111.379) (width 0.25) (layer F.Cu) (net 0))
 (segment (start 167.650701 96.819128) (end 167.659728 96.819128) (width 0.25) (layer F.Cu) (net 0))
 (segment (start 167.659728 96.819128) (end 172.3644 101.5238) (width 0.25) (layer F.Cu) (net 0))
 (segment (start 172.3644 101.5238) (end 172.3644 102.0064) (width 0.25) (layer F.Cu) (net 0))
 (segment (start 172.3644 102.0064) (end 172.7962 102.4382) (width 0.25) (layer F.Cu) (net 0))
 (segment (start 172.7962 102.4382) (end 172.7962 104.3686) (width 0.25) (layer F.Cu) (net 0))
 (segment (start 172.7962 104.3686) (end 173.2534 104.8258) (width 0.25) (layer F.Cu) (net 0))
 (segment (start 173.2534 104.8258) (end 173.2534 106.7054) (width 0.25) (layer F.Cu) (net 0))
 (segment (start 173.2534 106.7054) (end 175.387 108.839) (width 0.25) (layer F.Cu) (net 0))
 (segment (start 168.216386 96.253443) (end 168.216386 96.258186) (width 0.25) (layer F.Cu) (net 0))
 (segment (start 168.216386 96.258186) (end 172.8216 100.8634) (width 0.25) (layer F.Cu) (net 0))
 (segment (start 172.8216 100.8634) (end 172.8216 101.8286) (width 0.25) (layer F.Cu) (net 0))
 (segment (start 172.8216 101.8286) (end 173.2534 102.2604) (width 0.25) (layer F.Cu) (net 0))
 (segment (start 173.2534 102.2604) (end 173.2534 104.1654) (width 0.25) (layer F.Cu) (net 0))
 (segment (start 173.2534 104.1654) (end 175.387 106.299) (width 0.25) (layer F.Cu) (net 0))
 (segment (start 167.085016 87.273187) (end 167.085016 87.270584) (width 0.25) (layer F.Cu) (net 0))
 (segment (start 167.085016 87.270584) (end 172.339 82.0166) (width 0.25) (layer F.Cu) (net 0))
 (segment (start 172.339 82.0166) (end 172.339 80.1116) (width 0.25) (layer F.Cu) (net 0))
 (segment (start 172.339 80.1116) (end 172.7962 79.6544) (width 0.25) (layer F.Cu) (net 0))
 (segment (start 172.7962 79.6544) (end 172.7962 77.7494) (width 0.25) (layer F.Cu) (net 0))
 (segment (start 172.7962 77.7494) (end 173.2534 77.2922) (width 0.25) (layer F.Cu) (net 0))
 (segment (start 173.2534 77.2922) (end 173.2534 75.4126) (width 0.25) (layer F.Cu) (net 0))
 (segment (start 173.2534 75.4126) (end 175.387 73.279) (width 0.25) (layer F.Cu) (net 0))
 (segment (start 167.650701 87.838872) (end 167.659728 87.838872) (width 0.25) (layer F.Cu) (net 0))
 (segment (start 167.659728 87.838872) (end 172.339 83.1596) (width 0.25) (layer F.Cu) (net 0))
 (segment (start 172.339 83.1596) (end 172.339 82.6516) (width 0.25) (layer F.Cu) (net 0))
 (segment (start 172.339 82.6516) (end 172.7962 82.1944) (width 0.25) (layer F.Cu) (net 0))
 (segment (start 172.7962 82.1944) (end 172.7962 80.3148) (width 0.25) (layer F.Cu) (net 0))
 (segment (start 172.7962 80.3148) (end 173.2534 79.8576) (width 0.25) (layer F.Cu) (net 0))
 (segment (start 173.2534 79.8576) (end 173.2534 77.9526) (width 0.25) (layer F.Cu) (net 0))
 (segment (start 173.2534 77.9526) (end 175.387 75.819) (width 0.25) (layer F.Cu) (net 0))
 (segment (start 168.216386 88.404557) (end 168.216386 88.399814) (width 0.25) (layer F.Cu) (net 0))
 (segment (start 168.216386 88.399814) (end 172.7962 83.82) (width 0.25) (layer F.Cu) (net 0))
 (segment (start 172.7962 83.82) (end 172.7962 82.8548) (width 0.25) (layer F.Cu) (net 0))
 (segment (start 172.7962 82.8548) (end 173.2534 82.3976) (width 0.25) (layer F.Cu) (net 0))
 (segment (start 173.2534 82.3976) (end 173.2534 80.4926) (width 0.25) (layer F.Cu) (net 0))
 (segment (start 173.2534 80.4926) (end 175.387 78.359) (width 0.25) (layer F.Cu) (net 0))
 (segment (start 163.195928 88.970243) (end 163.189043 88.970243) (width 0.25) (layer F.Cu) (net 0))
 (segment (start 163.189043 88.970243) (end 158.7246 84.5058) (width 0.25) (layer F.Cu) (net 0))
 (segment (start 158.7246 84.5058) (end 158.7246 83.0326) (width 0.25) (layer F.Cu) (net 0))
 (segment (start 158.7246 83.0326) (end 156.591 80.899) (width 0.25) (layer F.Cu) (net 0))
 (segment (start 163.195928 95.687757) (end 163.189043 95.687757) (width 0.25) (layer F.Cu) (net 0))
 (segment (start 163.189043 95.687757) (end 158.6992 100.1776) (width 0.25) (layer F.Cu) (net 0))
 (segment (start 158.6992 100.1776) (end 158.6992 101.6508) (width 0.25) (layer F.Cu) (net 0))
 (segment (start 158.6992 101.6508) (end 156.591 103.759) (width 0.25) (layer F.Cu) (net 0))
 (segment (start 168.782072 95.687757) (end 168.788957 95.687757) (width 0.25) (layer F.Cu) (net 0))
 (segment (start 168.788957 95.687757) (end 173.2788 100.1776) (width 0.25) (layer F.Cu) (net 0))
 (segment (start 173.2788 100.1776) (end 173.2788 101.6508) (width 0.25) (layer F.Cu) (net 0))
 (segment (start 173.2788 101.6508) (end 175.387 103.759) (width 0.25) (layer F.Cu) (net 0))
 (segment (start 168.782072 88.970243) (end 168.788957 88.970243) (width 0.25) (layer F.Cu) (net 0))
 (segment (start 168.788957 88.970243) (end 173.2534 84.5058) (width 0.25) (layer F.Cu) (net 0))
 (segment (start 173.2534 84.5058) (end 173.2534 83.0326) (width 0.25) (layer F.Cu) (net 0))
 (segment (start 173.2534 83.0326) (end 175.387 80.899) (width 0.25) (layer F.Cu) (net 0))
 (segment (start 156.591 83.439) (end 156.591 83.496685) (width 0.25) (layer F.Cu) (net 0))
 (segment (start 156.591 83.496685) (end 162.630243 89.535928) (width 0.25) (layer F.Cu) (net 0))
 (segment (start 156.591 85.979) (end 157.941943 85.979) (width 0.25) (layer F.Cu) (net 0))
 (segment (start 157.941943 85.979) (end 162.064557 90.101614) (width 0.25) (layer F.Cu) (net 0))
 (segment (start 156.591 88.519) (end 159.350573 88.519) (width 0.25) (layer F.Cu) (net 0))
 (segment (start 159.350573 88.519) (end 161.498872 90.667299) (width 0.25) (layer F.Cu) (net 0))
 (segment (start 156.591 101.219) (end 156.591 101.161315) (width 0.25) (layer F.Cu) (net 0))
 (segment (start 156.591 101.161315) (end 162.630243 95.122072) (width 0.25) (layer F.Cu) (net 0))
 (segment (start 156.591 98.679) (end 157.941943 98.679) (width 0.25) (layer F.Cu) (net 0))
 (segment (start 157.941943 98.679) (end 162.064557 94.556386) (width 0.25) (layer F.Cu) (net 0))
 (segment (start 156.591 96.139) (end 159.350573 96.139) (width 0.25) (layer F.Cu) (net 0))
 (segment (start 159.350573 96.139) (end 161.498872 93.990701) (width 0.25) (layer F.Cu) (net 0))
 (segment (start 160.933187 93.425016) (end 156.764984 93.425016) (width 0.25) (layer F.Cu) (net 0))
 (segment (start 156.764984 93.425016) (end 156.591 93.599) (width 0.25) (layer F.Cu) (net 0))
 (segment (start 160.933187 91.232984) (end 156.764984 91.232984) (width 0.25) (layer F.Cu) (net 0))
 (segment (start 156.764984 91.232984) (end 156.591 91.059) (width 0.25) (layer F.Cu) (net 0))
 (segment (start 175.387 83.439) (end 175.387 83.496685) (width 0.25) (layer F.Cu) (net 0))
 (segment (start 175.387 83.496685) (end 169.347757 89.535928) (width 0.25) (layer F.Cu) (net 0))
 (segment (start 175.387 101.219) (end 175.387 101.161315) (width 0.25) (layer F.Cu) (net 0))
 (segment (start 175.387 101.161315) (end 169.347757 95.122072) (width 0.25) (layer F.Cu) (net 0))
 (segment (start 175.387 98.679) (end 174.036057 98.679) (width 0.25) (layer F.Cu) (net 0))
 (segment (start 174.036057 98.679) (end 169.913443 94.556386) (width 0.25) (layer F.Cu) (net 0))
 (segment (start 175.387 96.139) (end 172.627427 96.139) (width 0.25) (layer F.Cu) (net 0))
 (segment (start 172.627427 96.139) (end 170.479128 93.990701) (width 0.25) (layer F.Cu) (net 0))
 (segment (start 171.044813 93.425016) (end 175.213016 93.425016) (width 0.25) (layer F.Cu) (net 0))
 (segment (start 175.213016 93.425016) (end 175.387 93.599) (width 0.25) (layer F.Cu) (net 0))
 (segment (start 175.387 85.979) (end 174.036057 85.979) (width 0.25) (layer F.Cu) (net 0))
 (segment (start 174.036057 85.979) (end 169.913443 90.101614) (width 0.25) (layer F.Cu) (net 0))
 (segment (start 175.387 88.519) (end 172.6438 88.519) (width 0.25) (layer F.Cu) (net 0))
 (segment (start 172.6438 88.519) (end 172.627427 88.519) (width 0.25) (layer F.Cu) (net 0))
 (segment (start 172.627427 88.519) (end 170.479128 90.667299) (width 0.25) (layer F.Cu) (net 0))
 (segment (start 171.044813 91.232984) (end 175.213016 91.232984) (width 0.25) (layer F.Cu) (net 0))
 (segment (start 175.213016 91.232984) (end 175.387 91.059) (width 0.25) (layer F.Cu) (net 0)))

